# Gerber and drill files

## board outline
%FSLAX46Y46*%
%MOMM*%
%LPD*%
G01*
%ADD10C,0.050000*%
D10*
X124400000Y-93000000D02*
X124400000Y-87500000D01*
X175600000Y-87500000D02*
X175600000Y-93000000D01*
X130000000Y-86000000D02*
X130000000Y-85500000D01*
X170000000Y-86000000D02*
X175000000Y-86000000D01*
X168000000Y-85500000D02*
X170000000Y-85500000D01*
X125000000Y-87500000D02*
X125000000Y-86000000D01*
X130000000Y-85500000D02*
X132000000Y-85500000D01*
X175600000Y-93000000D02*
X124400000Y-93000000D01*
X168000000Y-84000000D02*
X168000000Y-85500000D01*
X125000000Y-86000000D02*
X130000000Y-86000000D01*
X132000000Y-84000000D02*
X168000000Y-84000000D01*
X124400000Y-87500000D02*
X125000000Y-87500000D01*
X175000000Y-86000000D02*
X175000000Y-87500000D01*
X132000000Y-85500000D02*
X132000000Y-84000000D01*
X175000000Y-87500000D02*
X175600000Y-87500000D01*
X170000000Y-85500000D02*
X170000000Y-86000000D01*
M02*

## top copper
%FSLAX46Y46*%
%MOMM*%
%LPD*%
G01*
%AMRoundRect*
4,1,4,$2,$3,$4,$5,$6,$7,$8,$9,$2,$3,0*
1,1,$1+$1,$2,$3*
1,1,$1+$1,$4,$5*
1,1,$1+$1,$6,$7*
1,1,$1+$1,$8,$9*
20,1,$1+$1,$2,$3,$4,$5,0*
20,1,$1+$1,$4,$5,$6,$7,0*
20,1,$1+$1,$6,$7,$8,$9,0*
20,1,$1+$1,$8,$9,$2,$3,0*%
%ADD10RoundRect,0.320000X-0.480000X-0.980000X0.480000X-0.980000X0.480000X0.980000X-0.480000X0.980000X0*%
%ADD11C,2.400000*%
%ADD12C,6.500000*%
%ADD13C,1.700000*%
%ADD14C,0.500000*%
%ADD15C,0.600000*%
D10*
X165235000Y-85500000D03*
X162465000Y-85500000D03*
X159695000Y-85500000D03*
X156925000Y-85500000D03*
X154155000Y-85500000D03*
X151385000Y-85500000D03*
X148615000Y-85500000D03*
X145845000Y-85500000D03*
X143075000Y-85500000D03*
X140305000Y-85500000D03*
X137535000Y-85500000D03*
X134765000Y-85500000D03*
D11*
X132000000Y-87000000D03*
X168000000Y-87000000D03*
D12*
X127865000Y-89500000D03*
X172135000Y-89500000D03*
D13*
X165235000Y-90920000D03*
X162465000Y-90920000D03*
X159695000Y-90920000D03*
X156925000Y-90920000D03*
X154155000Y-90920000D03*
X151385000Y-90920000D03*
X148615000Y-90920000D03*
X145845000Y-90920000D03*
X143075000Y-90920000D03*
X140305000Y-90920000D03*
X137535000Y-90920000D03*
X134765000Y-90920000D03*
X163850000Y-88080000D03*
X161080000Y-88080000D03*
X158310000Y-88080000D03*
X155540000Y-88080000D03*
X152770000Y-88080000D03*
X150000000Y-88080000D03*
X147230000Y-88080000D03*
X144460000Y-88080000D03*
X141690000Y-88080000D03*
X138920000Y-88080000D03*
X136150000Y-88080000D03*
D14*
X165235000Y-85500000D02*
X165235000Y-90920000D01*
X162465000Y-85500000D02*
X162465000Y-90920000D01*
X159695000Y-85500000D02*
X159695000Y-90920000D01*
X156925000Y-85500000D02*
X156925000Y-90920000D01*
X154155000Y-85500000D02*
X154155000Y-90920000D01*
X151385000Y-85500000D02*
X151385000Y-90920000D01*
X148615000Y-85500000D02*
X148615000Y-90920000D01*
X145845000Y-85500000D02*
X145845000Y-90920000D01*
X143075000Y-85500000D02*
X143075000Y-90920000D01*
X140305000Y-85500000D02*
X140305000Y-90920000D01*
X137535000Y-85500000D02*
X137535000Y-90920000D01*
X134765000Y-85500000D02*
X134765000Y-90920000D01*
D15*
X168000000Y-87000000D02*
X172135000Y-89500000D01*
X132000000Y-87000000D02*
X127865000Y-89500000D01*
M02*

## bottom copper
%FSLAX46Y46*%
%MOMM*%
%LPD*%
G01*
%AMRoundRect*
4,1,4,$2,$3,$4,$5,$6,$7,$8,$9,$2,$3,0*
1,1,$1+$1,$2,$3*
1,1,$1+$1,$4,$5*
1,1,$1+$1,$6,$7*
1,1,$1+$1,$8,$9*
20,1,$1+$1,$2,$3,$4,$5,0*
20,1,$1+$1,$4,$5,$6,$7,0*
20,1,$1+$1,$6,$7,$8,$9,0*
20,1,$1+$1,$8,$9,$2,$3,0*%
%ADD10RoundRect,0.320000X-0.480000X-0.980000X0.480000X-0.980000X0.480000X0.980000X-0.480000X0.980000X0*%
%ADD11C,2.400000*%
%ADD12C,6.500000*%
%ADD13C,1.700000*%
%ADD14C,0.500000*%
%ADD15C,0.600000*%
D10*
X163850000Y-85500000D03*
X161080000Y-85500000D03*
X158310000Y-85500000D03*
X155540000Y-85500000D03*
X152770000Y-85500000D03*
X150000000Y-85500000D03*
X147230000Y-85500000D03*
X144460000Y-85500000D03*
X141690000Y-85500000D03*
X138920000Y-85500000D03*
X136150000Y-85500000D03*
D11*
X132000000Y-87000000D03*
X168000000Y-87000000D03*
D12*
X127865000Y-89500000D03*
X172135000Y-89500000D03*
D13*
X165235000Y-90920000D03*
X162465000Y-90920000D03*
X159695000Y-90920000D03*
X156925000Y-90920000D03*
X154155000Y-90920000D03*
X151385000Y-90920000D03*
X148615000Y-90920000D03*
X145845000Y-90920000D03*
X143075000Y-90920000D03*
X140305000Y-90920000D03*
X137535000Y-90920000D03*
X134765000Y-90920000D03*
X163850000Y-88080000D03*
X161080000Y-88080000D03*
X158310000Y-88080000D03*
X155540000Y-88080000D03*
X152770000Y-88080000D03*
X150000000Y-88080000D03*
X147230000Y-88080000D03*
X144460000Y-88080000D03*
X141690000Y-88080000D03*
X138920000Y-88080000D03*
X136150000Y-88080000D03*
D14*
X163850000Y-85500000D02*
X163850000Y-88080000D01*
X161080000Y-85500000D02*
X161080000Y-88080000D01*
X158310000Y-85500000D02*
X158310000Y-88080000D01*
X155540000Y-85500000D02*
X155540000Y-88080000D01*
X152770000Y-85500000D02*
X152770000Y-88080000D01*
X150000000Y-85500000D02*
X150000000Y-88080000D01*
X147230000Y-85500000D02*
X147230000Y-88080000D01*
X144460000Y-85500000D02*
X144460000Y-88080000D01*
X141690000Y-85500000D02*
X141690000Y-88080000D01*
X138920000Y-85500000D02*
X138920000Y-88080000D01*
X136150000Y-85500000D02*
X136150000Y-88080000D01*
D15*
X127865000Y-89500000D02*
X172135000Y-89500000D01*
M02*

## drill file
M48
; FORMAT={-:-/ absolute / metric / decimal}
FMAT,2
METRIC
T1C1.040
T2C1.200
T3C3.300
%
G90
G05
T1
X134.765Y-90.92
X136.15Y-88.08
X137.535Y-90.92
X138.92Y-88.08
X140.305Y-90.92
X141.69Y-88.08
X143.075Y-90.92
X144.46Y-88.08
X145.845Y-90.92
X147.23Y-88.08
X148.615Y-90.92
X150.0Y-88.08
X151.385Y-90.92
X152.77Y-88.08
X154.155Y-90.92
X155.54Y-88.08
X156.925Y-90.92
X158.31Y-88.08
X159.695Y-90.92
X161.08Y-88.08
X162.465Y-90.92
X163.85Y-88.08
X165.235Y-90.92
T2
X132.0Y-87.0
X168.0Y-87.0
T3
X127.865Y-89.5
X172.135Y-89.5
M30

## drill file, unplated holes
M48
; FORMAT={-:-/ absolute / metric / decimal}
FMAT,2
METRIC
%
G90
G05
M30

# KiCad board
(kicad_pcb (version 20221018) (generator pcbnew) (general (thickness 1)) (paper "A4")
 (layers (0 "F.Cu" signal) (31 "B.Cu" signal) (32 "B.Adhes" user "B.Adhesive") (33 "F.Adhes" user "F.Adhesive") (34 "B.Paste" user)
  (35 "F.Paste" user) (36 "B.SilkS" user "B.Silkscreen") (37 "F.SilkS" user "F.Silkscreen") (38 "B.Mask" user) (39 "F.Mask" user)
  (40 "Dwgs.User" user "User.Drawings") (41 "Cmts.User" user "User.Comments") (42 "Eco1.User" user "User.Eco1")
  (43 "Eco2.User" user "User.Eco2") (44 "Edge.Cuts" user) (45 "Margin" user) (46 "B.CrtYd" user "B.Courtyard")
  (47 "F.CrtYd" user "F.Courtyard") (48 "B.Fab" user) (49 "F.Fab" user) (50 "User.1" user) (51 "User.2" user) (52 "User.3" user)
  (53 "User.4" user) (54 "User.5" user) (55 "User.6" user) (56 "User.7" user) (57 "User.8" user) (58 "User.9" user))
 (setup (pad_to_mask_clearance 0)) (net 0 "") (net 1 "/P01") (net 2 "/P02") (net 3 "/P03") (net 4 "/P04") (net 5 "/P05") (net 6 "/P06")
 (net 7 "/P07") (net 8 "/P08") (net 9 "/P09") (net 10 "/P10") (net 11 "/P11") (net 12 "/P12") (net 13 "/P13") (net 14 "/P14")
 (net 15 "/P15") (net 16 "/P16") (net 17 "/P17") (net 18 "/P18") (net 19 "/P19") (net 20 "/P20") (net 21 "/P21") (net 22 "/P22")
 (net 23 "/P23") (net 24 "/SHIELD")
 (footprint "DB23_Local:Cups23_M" (layer "F.Cu") (at 150 80)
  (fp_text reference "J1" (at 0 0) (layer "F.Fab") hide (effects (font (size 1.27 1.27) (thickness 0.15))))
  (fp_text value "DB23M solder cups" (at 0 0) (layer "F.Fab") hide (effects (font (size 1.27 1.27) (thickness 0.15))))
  (pad "1" smd roundrect (at 15.235 5.5) (size 1.6 2.6) (layers "F.Cu" "F.Mask") (roundrect_rratio 0.2) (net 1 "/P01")
   (thermal_bridge_angle 45))
  (pad "2" smd roundrect (at 12.465 5.5) (size 1.6 2.6) (layers "F.Cu" "F.Mask") (roundrect_rratio 0.2) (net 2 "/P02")
   (thermal_bridge_angle 45))
  (pad "3" smd roundrect (at 9.695 5.5) (size 1.6 2.6) (layers "F.Cu" "F.Mask") (roundrect_rratio 0.2) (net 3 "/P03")
   (thermal_bridge_angle 45))
  (pad "4" smd roundrect (at 6.925 5.5) (size 1.6 2.6) (layers "F.Cu" "F.Mask") (roundrect_rratio 0.2) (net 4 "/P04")
   (thermal_bridge_angle 45))
  (pad "5" smd roundrect (at 4.155 5.5) (size 1.6 2.6) (layers "F.Cu" "F.Mask") (roundrect_rratio 0.2) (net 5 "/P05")
   (thermal_bridge_angle 45))
  (pad "6" smd roundrect (at 1.385 5.5) (size 1.6 2.6) (layers "F.Cu" "F.Mask") (roundrect_rratio 0.2) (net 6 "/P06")
   (thermal_bridge_angle 45))
  (pad "7" smd roundrect (at -1.385 5.5) (size 1.6 2.6) (layers "F.Cu" "F.Mask") (roundrect_rratio 0.2) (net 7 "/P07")
   (thermal_bridge_angle 45))
  (pad "8" smd roundrect (at -4.155 5.5) (size 1.6 2.6) (layers "F.Cu" "F.Mask") (roundrect_rratio 0.2) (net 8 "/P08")
   (thermal_bridge_angle 45))
  (pad "9" smd roundrect (at -6.925 5.5) (size 1.6 2.6) (layers "F.Cu" "F.Mask") (roundrect_rratio 0.2) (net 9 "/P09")
   (thermal_bridge_angle 45))
  (pad "10" smd roundrect (at -9.695 5.5) (size 1.6 2.6) (layers "F.Cu" "F.Mask") (roundrect_rratio 0.2) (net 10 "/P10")
   (thermal_bridge_angle 45))
  (pad "11" smd roundrect (at -12.465 5.5) (size 1.6 2.6) (layers "F.Cu" "F.Mask") (roundrect_rratio 0.2) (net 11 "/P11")
   (thermal_bridge_angle 45))
  (pad "12" smd roundrect (at -15.235 5.5) (size 1.6 2.6) (layers "F.Cu" "F.Mask") (roundrect_rratio 0.2) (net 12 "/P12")
   (thermal_bridge_angle 45))
  (pad "13" smd roundrect (at 13.85 5.5) (size 1.6 2.6) (layers "B.Cu" "B.Mask") (roundrect_rratio 0.2) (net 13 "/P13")
   (thermal_bridge_angle 45))
  (pad "14" smd roundrect (at 11.08 5.5) (size 1.6 2.6) (layers "B.Cu" "B.Mask") (roundrect_rratio 0.2) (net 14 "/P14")
   (thermal_bridge_angle 45))
  (pad "15" smd roundrect (at 8.31 5.5) (size 1.6 2.6) (layers "B.Cu" "B.Mask") (roundrect_rratio 0.2) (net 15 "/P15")
   (thermal_bridge_angle 45))
  (pad "16" smd roundrect (at 5.54 5.5) (size 1.6 2.6) (layers "B.Cu" "B.Mask") (roundrect_rratio 0.2) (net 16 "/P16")
   (thermal_bridge_angle 45))
  (pad "17" smd roundrect (at 2.77 5.5) (size 1.6 2.6) (layers "B.Cu" "B.Mask") (roundrect_rratio 0.2) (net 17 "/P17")
   (thermal_bridge_angle 45))
  (pad "18" smd roundrect (at 0 5.5) (size 1.6 2.6) (layers "B.Cu" "B.Mask") (roundrect_rratio 0.2) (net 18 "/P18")
   (thermal_bridge_angle 45))
  (pad "19" smd roundrect (at -2.77 5.5) (size 1.6 2.6) (layers "B.Cu" "B.Mask") (roundrect_rratio 0.2) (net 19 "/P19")
   (thermal_bridge_angle 45))
  (pad "20" smd roundrect (at -5.54 5.5) (size 1.6 2.6) (layers "B.Cu" "B.Mask") (roundrect_rratio 0.2) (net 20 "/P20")
   (thermal_bridge_angle 45))
  (pad "21" smd roundrect (at -8.31 5.5) (size 1.6 2.6) (layers "B.Cu" "B.Mask") (roundrect_rratio 0.2) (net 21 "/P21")
   (thermal_bridge_angle 45))
  (pad "22" smd roundrect (at -11.08 5.5) (size 1.6 2.6) (layers "B.Cu" "B.Mask") (roundrect_rratio 0.2) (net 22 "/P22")
   (thermal_bridge_angle 45))
  (pad "23" smd roundrect (at -13.85 5.5) (size 1.6 2.6) (layers "B.Cu" "B.Mask") (roundrect_rratio 0.2) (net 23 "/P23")
   (thermal_bridge_angle 45)))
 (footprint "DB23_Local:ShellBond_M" (layer "F.Cu") (at 150 80)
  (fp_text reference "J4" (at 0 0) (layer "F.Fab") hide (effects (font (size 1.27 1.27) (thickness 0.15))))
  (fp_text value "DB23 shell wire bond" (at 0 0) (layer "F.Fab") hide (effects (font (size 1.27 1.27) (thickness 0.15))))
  (pad "1" thru_hole circle (at -18 7) (size 2.4 2.4) (drill 1.2) (layers "*.Cu" "*.Mask") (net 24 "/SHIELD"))
  (pad "2" thru_hole circle (at 18 7) (size 2.4 2.4) (drill 1.2) (layers "*.Cu" "*.Mask") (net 24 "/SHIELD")))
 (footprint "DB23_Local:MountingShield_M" (layer "F.Cu") (at 150 80)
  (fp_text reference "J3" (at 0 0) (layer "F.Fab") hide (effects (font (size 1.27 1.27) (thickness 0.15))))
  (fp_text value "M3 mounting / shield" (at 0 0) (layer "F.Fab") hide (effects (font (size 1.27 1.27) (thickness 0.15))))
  (pad "1" thru_hole circle (at -22.135 9.5) (size 6.5 6.5) (drill 3.3) (layers "*.Cu" "*.Mask") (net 24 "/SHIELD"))
  (pad "2" thru_hole circle (at 22.135 9.5) (size 6.5 6.5) (drill 3.3) (layers "*.Cu" "*.Mask") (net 24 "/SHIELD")))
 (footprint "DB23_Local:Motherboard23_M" (layer "F.Cu") (at 150 80)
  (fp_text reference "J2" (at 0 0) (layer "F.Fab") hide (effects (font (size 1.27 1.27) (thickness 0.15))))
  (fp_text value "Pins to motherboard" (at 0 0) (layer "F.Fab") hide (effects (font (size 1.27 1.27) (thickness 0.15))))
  (pad "1" thru_hole circle (at 15.235 10.92) (size 1.7 1.7) (drill 1.04) (layers "*.Cu" "*.Mask") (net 1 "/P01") (thermal_bridge_angle 45))
  (pad "2" thru_hole circle (at 12.465 10.92) (size 1.7 1.7) (drill 1.04) (layers "*.Cu" "*.Mask") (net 2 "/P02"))
  (pad "3" thru_hole circle (at 9.695 10.92) (size 1.7 1.7) (drill 1.04) (layers "*.Cu" "*.Mask") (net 3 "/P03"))
  (pad "4" thru_hole circle (at 6.925 10.92) (size 1.7 1.7) (drill 1.04) (layers "*.Cu" "*.Mask") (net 4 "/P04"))
  (pad "5" thru_hole circle (at 4.155 10.92) (size 1.7 1.7) (drill 1.04) (layers "*.Cu" "*.Mask") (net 5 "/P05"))
  (pad "6" thru_hole circle (at 1.385 10.92) (size 1.7 1.7) (drill 1.04) (layers "*.Cu" "*.Mask") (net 6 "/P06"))
  (pad "7" thru_hole circle (at -1.385 10.92) (size 1.7 1.7) (drill 1.04) (layers "*.Cu" "*.Mask") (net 7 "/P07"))
  (pad "8" thru_hole circle (at -4.155 10.92) (size 1.7 1.7) (drill 1.04) (layers "*.Cu" "*.Mask") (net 8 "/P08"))
  (pad "9" thru_hole circle (at -6.925 10.92) (size 1.7 1.7) (drill 1.04) (layers "*.Cu" "*.Mask") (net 9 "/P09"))
  (pad "10" thru_hole circle (at -9.695 10.92) (size 1.7 1.7) (drill 1.04) (layers "*.Cu" "*.Mask") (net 10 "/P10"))
  (pad "11" thru_hole circle (at -12.465 10.92) (size 1.7 1.7) (drill 1.04) (layers "*.Cu" "*.Mask") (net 11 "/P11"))
  (pad "12" thru_hole circle (at -15.235 10.92) (size 1.7 1.7) (drill 1.04) (layers "*.Cu" "*.Mask") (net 12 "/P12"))
  (pad "13" thru_hole circle (at 13.85 8.08) (size 1.7 1.7) (drill 1.04) (layers "*.Cu" "*.Mask") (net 13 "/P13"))
  (pad "14" thru_hole circle (at 11.08 8.08) (size 1.7 1.7) (drill 1.04) (layers "*.Cu" "*.Mask") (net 14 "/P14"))
  (pad "15" thru_hole circle (at 8.31 8.08) (size 1.7 1.7) (drill 1.04) (layers "*.Cu" "*.Mask") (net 15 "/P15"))
  (pad "16" thru_hole circle (at 5.54 8.08) (size 1.7 1.7) (drill 1.04) (layers "*.Cu" "*.Mask") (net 16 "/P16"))
  (pad "17" thru_hole circle (at 2.77 8.08) (size 1.7 1.7) (drill 1.04) (layers "*.Cu" "*.Mask") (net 17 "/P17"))
  (pad "18" thru_hole circle (at 0 8.08) (size 1.7 1.7) (drill 1.04) (layers "*.Cu" "*.Mask") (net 18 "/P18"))
  (pad "19" thru_hole circle (at -2.77 8.08) (size 1.7 1.7) (drill 1.04) (layers "*.Cu" "*.Mask") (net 19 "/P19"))
  (pad "20" thru_hole circle (at -5.54 8.08) (size 1.7 1.7) (drill 1.04) (layers "*.Cu" "*.Mask") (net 20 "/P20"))
  (pad "21" thru_hole circle (at -8.31 8.08) (size 1.7 1.7) (drill 1.04) (layers "*.Cu" "*.Mask") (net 21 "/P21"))
  (pad "22" thru_hole circle (at -11.08 8.08) (size 1.7 1.7) (drill 1.04) (layers "*.Cu" "*.Mask") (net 22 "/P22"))
  (pad "23" thru_hole circle (at -13.85 8.08) (size 1.7 1.7) (drill 1.04) (layers "*.Cu" "*.Mask") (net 23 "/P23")))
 (gr_line (start 124.4 93) (end 124.4 87.5) (stroke (width 0.05) (type default)) (layer "Edge.Cuts"))
 (gr_line (start 175.6 87.5) (end 175.6 93) (stroke (width 0.05) (type default)) (layer "Edge.Cuts"))
 (gr_line (start 130 86) (end 130 85.5) (stroke (width 0.05) (type default)) (layer "Edge.Cuts"))
 (gr_line (start 170 86) (end 175 86) (stroke (width 0.05) (type default)) (layer "Edge.Cuts"))
 (gr_line (start 168 85.5) (end 170 85.5) (stroke (width 0.05) (type default)) (layer "Edge.Cuts"))
 (gr_line (start 125 87.5) (end 125 86) (stroke (width 0.05) (type default)) (layer "Edge.Cuts"))
 (gr_line (start 130 85.5) (end 132 85.5) (stroke (width 0.05) (type default)) (layer "Edge.Cuts"))
 (gr_line (start 175.6 93) (end 124.4 93) (stroke (width 0.05) (type default)) (layer "Edge.Cuts"))
 (gr_line (start 168 84) (end 168 85.5) (stroke (width 0.05) (type default)) (layer "Edge.Cuts"))
 (gr_line (start 125 86) (end 130 86) (stroke (width 0.05) (type default)) (layer "Edge.Cuts"))
 (gr_line (start 132 84) (end 168 84) (stroke (width 0.05) (type default)) (layer "Edge.Cuts"))
 (gr_line (start 124.4 87.5) (end 125 87.5) (stroke (width 0.05) (type default)) (layer "Edge.Cuts"))
 (gr_line (start 175 86) (end 175 87.5) (stroke (width 0.05) (type default)) (layer "Edge.Cuts"))
 (gr_line (start 132 85.5) (end 132 84) (stroke (width 0.05) (type default)) (layer "Edge.Cuts"))
 (gr_line (start 175 87.5) (end 175.6 87.5) (stroke (width 0.05) (type default)) (layer "Edge.Cuts"))
 (gr_line (start 170 85.5) (end 170 86) (stroke (width 0.05) (type default)) (layer "Edge.Cuts"))
 (segment (start 165.235 85.5) (end 165.235 90.92) (width 0.5) (layer "F.Cu") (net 1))
 (segment (start 162.465 85.5) (end 162.465 90.92) (width 0.5) (layer "F.Cu") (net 2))
 (segment (start 159.695 85.5) (end 159.695 90.92) (width 0.5) (layer "F.Cu") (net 3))
 (segment (start 156.925 85.5) (end 156.925 90.92) (width 0.5) (layer "F.Cu") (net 4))
 (segment (start 154.155 85.5) (end 154.155 90.92) (width 0.5) (layer "F.Cu") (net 5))
 (segment (start 151.385 85.5) (end 151.385 90.92) (width 0.5) (layer "F.Cu") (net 6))
 (segment (start 148.615 85.5) (end 148.615 90.92) (width 0.5) (layer "F.Cu") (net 7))
 (segment (start 145.845 85.5) (end 145.845 90.92) (width 0.5) (layer "F.Cu") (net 8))
 (segment (start 143.075 85.5) (end 143.075 90.92) (width 0.5) (layer "F.Cu") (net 9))
 (segment (start 140.305 85.5) (end 140.305 90.92) (width 0.5) (layer "F.Cu") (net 10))
 (segment (start 137.535 85.5) (end 137.535 90.92) (width 0.5) (layer "F.Cu") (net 11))
 (segment (start 134.765 85.5) (end 134.765 90.92) (width 0.5) (layer "F.Cu") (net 12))
 (segment (start 163.85 85.5) (end 163.85 88.08) (width 0.5) (layer "B.Cu") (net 13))
 (segment (start 161.08 85.5) (end 161.08 88.08) (width 0.5) (layer "B.Cu") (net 14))
 (segment (start 158.31 85.5) (end 158.31 88.08) (width 0.5) (layer "B.Cu") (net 15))
 (segment (start 155.54 85.5) (end 155.54 88.08) (width 0.5) (layer "B.Cu") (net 16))
 (segment (start 152.77 85.5) (end 152.77 88.08) (width 0.5) (layer "B.Cu") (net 17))
 (segment (start 150 85.5) (end 150 88.08) (width 0.5) (layer "B.Cu") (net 18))
 (segment (start 147.23 85.5) (end 147.23 88.08) (width 0.5) (layer "B.Cu") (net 19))
 (segment (start 144.46 85.5) (end 144.46 88.08) (width 0.5) (layer "B.Cu") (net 20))
 (segment (start 141.69 85.5) (end 141.69 88.08) (width 0.5) (layer "B.Cu") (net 21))
 (segment (start 138.92 85.5) (end 138.92 88.08) (width 0.5) (layer "B.Cu") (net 22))
 (segment (start 136.15 85.5) (end 136.15 88.08) (width 0.5) (layer "B.Cu") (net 23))
 (segment (start 168 87) (end 172.135 89.5) (width 0.6) (layer "F.Cu") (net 24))
 (segment (start 132 87) (end 127.865 89.5) (width 0.6) (layer "F.Cu") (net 24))
 (segment (start 127.865 89.5) (end 172.135 89.5) (width 0.6) (layer "B.Cu") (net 24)))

